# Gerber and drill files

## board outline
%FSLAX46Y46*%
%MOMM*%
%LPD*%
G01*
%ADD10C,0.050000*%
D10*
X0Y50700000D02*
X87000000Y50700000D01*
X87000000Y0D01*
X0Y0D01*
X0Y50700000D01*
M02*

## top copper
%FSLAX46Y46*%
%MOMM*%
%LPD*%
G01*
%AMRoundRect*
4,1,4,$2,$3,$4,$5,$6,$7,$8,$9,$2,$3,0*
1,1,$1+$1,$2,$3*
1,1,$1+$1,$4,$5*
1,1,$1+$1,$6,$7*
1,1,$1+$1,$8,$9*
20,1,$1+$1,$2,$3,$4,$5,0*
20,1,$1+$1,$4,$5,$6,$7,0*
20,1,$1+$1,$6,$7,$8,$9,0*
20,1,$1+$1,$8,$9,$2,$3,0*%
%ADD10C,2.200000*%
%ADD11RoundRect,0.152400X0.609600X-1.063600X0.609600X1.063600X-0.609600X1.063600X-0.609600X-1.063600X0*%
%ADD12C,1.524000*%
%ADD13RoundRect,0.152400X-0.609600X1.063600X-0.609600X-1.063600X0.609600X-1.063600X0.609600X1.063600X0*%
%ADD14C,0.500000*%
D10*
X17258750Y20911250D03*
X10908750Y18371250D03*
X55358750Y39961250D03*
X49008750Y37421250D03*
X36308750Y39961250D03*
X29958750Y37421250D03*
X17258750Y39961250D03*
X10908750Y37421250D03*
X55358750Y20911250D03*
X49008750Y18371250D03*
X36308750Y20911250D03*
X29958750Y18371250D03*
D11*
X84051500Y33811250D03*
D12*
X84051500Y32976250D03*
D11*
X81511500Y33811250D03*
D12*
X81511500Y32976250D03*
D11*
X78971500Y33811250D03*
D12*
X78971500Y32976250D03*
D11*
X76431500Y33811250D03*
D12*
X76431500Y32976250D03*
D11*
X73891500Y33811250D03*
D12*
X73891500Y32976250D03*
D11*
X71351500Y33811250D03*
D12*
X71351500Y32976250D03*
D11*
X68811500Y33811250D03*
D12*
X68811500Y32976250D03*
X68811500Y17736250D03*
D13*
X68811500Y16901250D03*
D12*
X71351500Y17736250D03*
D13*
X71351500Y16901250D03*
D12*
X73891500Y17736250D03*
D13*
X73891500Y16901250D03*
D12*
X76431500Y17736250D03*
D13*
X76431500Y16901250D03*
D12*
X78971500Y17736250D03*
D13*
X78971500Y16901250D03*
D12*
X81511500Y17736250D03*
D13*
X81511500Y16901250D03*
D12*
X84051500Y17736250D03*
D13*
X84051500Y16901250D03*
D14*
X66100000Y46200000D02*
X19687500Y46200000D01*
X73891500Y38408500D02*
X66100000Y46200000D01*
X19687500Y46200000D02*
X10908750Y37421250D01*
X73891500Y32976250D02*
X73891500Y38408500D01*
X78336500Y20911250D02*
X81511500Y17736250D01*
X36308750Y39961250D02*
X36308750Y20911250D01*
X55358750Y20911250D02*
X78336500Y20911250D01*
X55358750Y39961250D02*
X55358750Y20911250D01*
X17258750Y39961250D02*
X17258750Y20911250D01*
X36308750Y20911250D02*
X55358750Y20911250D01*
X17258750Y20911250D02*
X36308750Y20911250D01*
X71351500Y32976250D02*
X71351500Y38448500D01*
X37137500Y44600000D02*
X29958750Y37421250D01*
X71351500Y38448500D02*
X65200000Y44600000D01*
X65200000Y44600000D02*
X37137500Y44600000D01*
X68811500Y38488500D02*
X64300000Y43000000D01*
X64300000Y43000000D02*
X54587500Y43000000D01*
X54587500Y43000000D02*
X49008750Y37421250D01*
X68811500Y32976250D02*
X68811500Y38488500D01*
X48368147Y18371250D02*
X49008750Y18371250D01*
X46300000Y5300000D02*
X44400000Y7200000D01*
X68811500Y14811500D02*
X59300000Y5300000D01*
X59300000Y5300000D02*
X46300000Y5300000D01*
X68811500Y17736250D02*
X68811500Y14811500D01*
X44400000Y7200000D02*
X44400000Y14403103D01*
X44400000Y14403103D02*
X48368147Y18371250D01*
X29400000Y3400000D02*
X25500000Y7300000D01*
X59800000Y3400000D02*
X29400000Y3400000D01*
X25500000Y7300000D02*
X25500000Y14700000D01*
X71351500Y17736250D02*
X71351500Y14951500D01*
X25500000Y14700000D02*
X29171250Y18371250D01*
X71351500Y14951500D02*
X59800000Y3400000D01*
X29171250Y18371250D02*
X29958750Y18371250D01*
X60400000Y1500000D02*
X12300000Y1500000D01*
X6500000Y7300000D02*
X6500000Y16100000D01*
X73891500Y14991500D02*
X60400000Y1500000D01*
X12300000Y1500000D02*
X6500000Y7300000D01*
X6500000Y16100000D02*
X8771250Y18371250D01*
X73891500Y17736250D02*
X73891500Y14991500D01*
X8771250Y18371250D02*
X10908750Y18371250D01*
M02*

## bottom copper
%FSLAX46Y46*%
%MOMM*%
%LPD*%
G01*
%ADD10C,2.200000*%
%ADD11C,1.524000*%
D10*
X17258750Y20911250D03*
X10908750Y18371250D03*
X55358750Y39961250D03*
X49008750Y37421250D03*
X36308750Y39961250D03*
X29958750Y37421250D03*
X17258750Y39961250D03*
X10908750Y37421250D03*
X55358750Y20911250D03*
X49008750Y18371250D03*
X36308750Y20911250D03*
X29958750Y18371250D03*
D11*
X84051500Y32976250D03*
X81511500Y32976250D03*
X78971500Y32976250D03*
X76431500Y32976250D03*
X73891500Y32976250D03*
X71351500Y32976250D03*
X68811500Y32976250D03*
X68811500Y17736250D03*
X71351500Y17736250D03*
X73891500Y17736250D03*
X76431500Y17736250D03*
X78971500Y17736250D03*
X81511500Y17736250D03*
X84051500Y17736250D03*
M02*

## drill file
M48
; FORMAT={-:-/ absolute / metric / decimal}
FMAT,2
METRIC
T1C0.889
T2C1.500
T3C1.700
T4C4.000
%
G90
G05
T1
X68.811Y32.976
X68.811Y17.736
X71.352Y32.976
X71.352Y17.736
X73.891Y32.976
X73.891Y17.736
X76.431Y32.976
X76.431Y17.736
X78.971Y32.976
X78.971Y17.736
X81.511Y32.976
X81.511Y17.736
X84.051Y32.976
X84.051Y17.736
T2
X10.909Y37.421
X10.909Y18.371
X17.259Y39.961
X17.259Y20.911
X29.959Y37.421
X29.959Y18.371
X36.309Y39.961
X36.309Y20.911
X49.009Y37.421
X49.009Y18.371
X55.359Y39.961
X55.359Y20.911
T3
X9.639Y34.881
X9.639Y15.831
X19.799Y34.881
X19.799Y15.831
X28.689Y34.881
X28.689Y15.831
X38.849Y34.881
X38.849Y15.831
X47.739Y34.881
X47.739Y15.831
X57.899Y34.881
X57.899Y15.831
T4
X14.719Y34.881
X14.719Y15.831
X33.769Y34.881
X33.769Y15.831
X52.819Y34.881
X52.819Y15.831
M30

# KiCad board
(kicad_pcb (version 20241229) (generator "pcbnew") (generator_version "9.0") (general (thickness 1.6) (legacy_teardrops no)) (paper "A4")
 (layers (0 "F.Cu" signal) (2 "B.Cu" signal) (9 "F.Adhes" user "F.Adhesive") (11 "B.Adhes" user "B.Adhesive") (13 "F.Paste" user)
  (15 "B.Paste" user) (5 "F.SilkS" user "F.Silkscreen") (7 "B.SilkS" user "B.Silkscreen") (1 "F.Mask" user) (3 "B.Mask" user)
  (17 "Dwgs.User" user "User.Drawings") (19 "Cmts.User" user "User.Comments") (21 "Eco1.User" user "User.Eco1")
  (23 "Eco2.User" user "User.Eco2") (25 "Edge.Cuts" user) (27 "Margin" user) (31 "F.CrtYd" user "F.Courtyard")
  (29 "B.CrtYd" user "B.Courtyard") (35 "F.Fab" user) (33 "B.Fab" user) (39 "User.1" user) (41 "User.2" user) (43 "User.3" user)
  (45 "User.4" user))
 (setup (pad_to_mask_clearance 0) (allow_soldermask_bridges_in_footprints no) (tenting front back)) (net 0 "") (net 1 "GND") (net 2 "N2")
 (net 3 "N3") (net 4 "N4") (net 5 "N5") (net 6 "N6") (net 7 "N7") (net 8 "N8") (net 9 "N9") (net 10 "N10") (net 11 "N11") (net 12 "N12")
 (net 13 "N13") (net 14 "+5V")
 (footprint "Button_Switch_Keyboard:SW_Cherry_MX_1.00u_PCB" (layer "F.Cu") (at 17.25875 -20.91125)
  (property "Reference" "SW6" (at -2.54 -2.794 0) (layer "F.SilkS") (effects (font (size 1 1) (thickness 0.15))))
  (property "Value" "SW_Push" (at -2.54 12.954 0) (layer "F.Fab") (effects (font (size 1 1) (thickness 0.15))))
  (pad "" np_thru_hole circle (at -7.62 5.08) (size 1.7 1.7) (drill 1.7) (layers "*.Cu" "*.Mask"))
  (pad "" np_thru_hole circle (at -2.54 5.08) (size 4 4) (drill 4) (layers "*.Cu" "*.Mask"))
  (pad "" np_thru_hole circle (at 2.54 5.08) (size 1.7 1.7) (drill 1.7) (layers "*.Cu" "*.Mask"))
  (pad "1" thru_hole circle (at 0 0) (size 2.2 2.2) (drill 1.5) (layers "*.Cu" "*.Mask") (remove_unused_layers no) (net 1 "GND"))
  (pad "2" thru_hole circle (at -6.35 2.54) (size 2.2 2.2) (drill 1.5) (layers "*.Cu" "*.Mask") (remove_unused_layers no) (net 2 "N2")))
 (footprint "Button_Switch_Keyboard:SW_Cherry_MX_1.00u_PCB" (layer "F.Cu") (at 55.35875 -39.96125)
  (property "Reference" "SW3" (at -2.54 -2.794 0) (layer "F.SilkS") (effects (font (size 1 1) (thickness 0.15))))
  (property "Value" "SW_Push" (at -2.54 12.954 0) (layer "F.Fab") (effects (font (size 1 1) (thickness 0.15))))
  (pad "" np_thru_hole circle (at -7.62 5.08) (size 1.7 1.7) (drill 1.7) (layers "*.Cu" "*.Mask"))
  (pad "" np_thru_hole circle (at -2.54 5.08) (size 4 4) (drill 4) (layers "*.Cu" "*.Mask"))
  (pad "" np_thru_hole circle (at 2.54 5.08) (size 1.7 1.7) (drill 1.7) (layers "*.Cu" "*.Mask"))
  (pad "1" thru_hole circle (at 0 0) (size 2.2 2.2) (drill 1.5) (layers "*.Cu" "*.Mask") (remove_unused_layers no) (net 1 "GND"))
  (pad "2" thru_hole circle (at -6.35 2.54) (size 2.2 2.2) (drill 1.5) (layers "*.Cu" "*.Mask") (remove_unused_layers no) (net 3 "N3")))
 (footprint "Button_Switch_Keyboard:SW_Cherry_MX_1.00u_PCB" (layer "F.Cu") (at 36.30875 -39.96125)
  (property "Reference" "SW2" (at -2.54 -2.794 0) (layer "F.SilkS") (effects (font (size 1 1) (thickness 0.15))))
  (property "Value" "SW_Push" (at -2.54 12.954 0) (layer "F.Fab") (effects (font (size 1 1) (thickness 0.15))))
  (pad "" np_thru_hole circle (at -7.62 5.08) (size 1.7 1.7) (drill 1.7) (layers "*.Cu" "*.Mask"))
  (pad "" np_thru_hole circle (at -2.54 5.08) (size 4 4) (drill 4) (layers "*.Cu" "*.Mask"))
  (pad "" np_thru_hole circle (at 2.54 5.08) (size 1.7 1.7) (drill 1.7) (layers "*.Cu" "*.Mask"))
  (pad "1" thru_hole circle (at 0 0) (size 2.2 2.2) (drill 1.5) (layers "*.Cu" "*.Mask") (remove_unused_layers no) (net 1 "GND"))
  (pad "2" thru_hole circle (at -6.35 2.54) (size 2.2 2.2) (drill 1.5) (layers "*.Cu" "*.Mask") (remove_unused_layers no) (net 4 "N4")))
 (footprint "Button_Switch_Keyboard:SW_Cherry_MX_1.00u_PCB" (layer "F.Cu") (at 17.25875 -39.96125)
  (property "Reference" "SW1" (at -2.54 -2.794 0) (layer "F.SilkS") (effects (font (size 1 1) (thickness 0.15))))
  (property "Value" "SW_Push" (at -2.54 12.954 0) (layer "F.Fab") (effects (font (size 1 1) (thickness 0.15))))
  (pad "" np_thru_hole circle (at -7.62 5.08) (size 1.7 1.7) (drill 1.7) (layers "*.Cu" "*.Mask"))
  (pad "" np_thru_hole circle (at -2.54 5.08) (size 4 4) (drill 4) (layers "*.Cu" "*.Mask"))
  (pad "" np_thru_hole circle (at 2.54 5.08) (size 1.7 1.7) (drill 1.7) (layers "*.Cu" "*.Mask"))
  (pad "1" thru_hole circle (at 0 0) (size 2.2 2.2) (drill 1.5) (layers "*.Cu" "*.Mask") (remove_unused_layers no) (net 1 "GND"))
  (pad "2" thru_hole circle (at -6.35 2.54) (size 2.2 2.2) (drill 1.5) (layers "*.Cu" "*.Mask") (remove_unused_layers no) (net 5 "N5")))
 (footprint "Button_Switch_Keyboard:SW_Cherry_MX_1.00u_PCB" (layer "F.Cu") (at 55.35875 -20.91125)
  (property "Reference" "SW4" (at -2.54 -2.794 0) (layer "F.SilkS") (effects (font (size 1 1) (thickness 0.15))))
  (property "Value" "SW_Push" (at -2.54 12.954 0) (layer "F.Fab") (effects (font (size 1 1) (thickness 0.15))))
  (pad "" np_thru_hole circle (at -7.62 5.08) (size 1.7 1.7) (drill 1.7) (layers "*.Cu" "*.Mask"))
  (pad "" np_thru_hole circle (at -2.54 5.08) (size 4 4) (drill 4) (layers "*.Cu" "*.Mask"))
  (pad "" np_thru_hole circle (at 2.54 5.08) (size 1.7 1.7) (drill 1.7) (layers "*.Cu" "*.Mask"))
  (pad "1" thru_hole circle (at 0 0) (size 2.2 2.2) (drill 1.5) (layers "*.Cu" "*.Mask") (remove_unused_layers no) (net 1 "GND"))
  (pad "2" thru_hole circle (at -6.35 2.54) (size 2.2 2.2) (drill 1.5) (layers "*.Cu" "*.Mask") (remove_unused_layers no) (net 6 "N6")))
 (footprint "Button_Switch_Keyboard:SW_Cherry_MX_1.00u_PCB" (layer "F.Cu") (at 36.30875 -20.91125)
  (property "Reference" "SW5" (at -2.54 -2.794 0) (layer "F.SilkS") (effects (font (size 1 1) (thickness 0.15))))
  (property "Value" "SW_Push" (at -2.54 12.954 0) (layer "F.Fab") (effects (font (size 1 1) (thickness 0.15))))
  (pad "" np_thru_hole circle (at -7.62 5.08) (size 1.7 1.7) (drill 1.7) (layers "*.Cu" "*.Mask"))
  (pad "" np_thru_hole circle (at -2.54 5.08) (size 4 4) (drill 4) (layers "*.Cu" "*.Mask"))
  (pad "" np_thru_hole circle (at 2.54 5.08) (size 1.7 1.7) (drill 1.7) (layers "*.Cu" "*.Mask"))
  (pad "1" thru_hole circle (at 0 0) (size 2.2 2.2) (drill 1.5) (layers "*.Cu" "*.Mask") (remove_unused_layers no) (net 1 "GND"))
  (pad "2" thru_hole circle (at -6.35 2.54) (size 2.2 2.2) (drill 1.5) (layers "*.Cu" "*.Mask") (remove_unused_layers no) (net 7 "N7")))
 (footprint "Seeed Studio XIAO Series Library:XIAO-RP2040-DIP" (layer "F.Cu") (at 76.4315 -25.35625 -90)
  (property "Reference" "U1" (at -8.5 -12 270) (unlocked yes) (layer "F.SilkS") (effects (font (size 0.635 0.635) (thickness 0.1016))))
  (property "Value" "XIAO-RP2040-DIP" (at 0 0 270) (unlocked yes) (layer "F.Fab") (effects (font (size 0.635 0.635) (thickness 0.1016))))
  (pad "1" smd roundrect (at -8.455 -7.62 90) (size 2.432 1.524) (layers "F.Cu" "F.Mask") (roundrect_rratio 0.1) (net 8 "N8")
   (thermal_bridge_angle 45))
  (pad "1" thru_hole circle (at -7.62 -7.62 90) (size 1.524 1.524) (drill 0.889) (layers "*.Cu" "*.Mask") (remove_unused_layers no)
   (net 8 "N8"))
  (pad "2" smd roundrect (at -8.455 -5.08 90) (size 2.432 1.524) (layers "F.Cu" "F.Mask") (roundrect_rratio 0.1) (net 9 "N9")
   (thermal_bridge_angle 45))
  (pad "2" thru_hole circle (at -7.62 -5.08 90) (size 1.524 1.524) (drill 0.889) (layers "*.Cu" "*.Mask") (remove_unused_layers no)
   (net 9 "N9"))
  (pad "3" smd roundrect (at -8.455 -2.54 90) (size 2.432 1.524) (layers "F.Cu" "F.Mask") (roundrect_rratio 0.1) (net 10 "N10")
   (thermal_bridge_angle 45))
  (pad "3" thru_hole circle (at -7.62 -2.54 90) (size 1.524 1.524) (drill 0.889) (layers "*.Cu" "*.Mask") (remove_unused_layers no)
   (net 10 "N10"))
  (pad "4" smd roundrect (at -8.455 0 90) (size 2.432 1.524) (layers "F.Cu" "F.Mask") (roundrect_rratio 0.1) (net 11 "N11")
   (thermal_bridge_angle 45))
  (pad "4" thru_hole circle (at -7.62 0 90) (size 1.524 1.524) (drill 0.889) (layers "*.Cu" "*.Mask") (remove_unused_layers no)
   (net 11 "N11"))
  (pad "5" smd roundrect (at -8.455 2.54 90) (size 2.432 1.524) (layers "F.Cu" "F.Mask") (roundrect_rratio 0.1) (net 5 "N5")
   (thermal_bridge_angle 45))
  (pad "5" thru_hole circle (at -7.62 2.54 90) (size 1.524 1.524) (drill 0.889) (layers "*.Cu" "*.Mask") (remove_unused_layers no)
   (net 5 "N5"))
  (pad "6" smd roundrect (at -8.455 5.08 90) (size 2.432 1.524) (layers "F.Cu" "F.Mask") (roundrect_rratio 0.1) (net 4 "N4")
   (thermal_bridge_angle 45))
  (pad "6" thru_hole circle (at -7.62 5.08 90) (size 1.524 1.524) (drill 0.889) (layers "*.Cu" "*.Mask") (remove_unused_layers no)
   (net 4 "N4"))
  (pad "7" smd roundrect (at -8.455 7.62 90) (size 2.432 1.524) (layers "F.Cu" "F.Mask") (roundrect_rratio 0.1) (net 3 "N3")
   (thermal_bridge_angle 45))
  (pad "7" thru_hole circle (at -7.62 7.62 90) (size 1.524 1.524) (drill 0.889) (layers "*.Cu" "*.Mask") (remove_unused_layers no)
   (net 3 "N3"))
  (pad "8" thru_hole circle (at 7.62 7.62 270) (size 1.524 1.524) (drill 0.889) (layers "*.Cu" "*.Mask") (remove_unused_layers no)
   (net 6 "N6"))
  (pad "8" smd roundrect (at 8.455 7.62 270) (size 2.432 1.524) (layers "F.Cu" "F.Mask") (roundrect_rratio 0.1) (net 6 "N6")
   (thermal_bridge_angle 45))
  (pad "9" thru_hole circle (at 7.62 5.08 270) (size 1.524 1.524) (drill 0.889) (layers "*.Cu" "*.Mask") (remove_unused_layers no)
   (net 7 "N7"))
  (pad "9" smd roundrect (at 8.455 5.08 270) (size 2.432 1.524) (layers "F.Cu" "F.Mask") (roundrect_rratio 0.1) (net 7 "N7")
   (thermal_bridge_angle 45))
  (pad "10" thru_hole circle (at 7.62 2.54 270) (size 1.524 1.524) (drill 0.889) (layers "*.Cu" "*.Mask") (remove_unused_layers no)
   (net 2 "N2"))
  (pad "10" smd roundrect (at 8.455 2.54 270) (size 2.432 1.524) (layers "F.Cu" "F.Mask") (roundrect_rratio 0.1) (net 2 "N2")
   (thermal_bridge_angle 45))
  (pad "11" thru_hole circle (at 7.62 0 270) (size 1.524 1.524) (drill 0.889) (layers "*.Cu" "*.Mask") (remove_unused_layers no)
   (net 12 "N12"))
  (pad "11" smd roundrect (at 8.455 0 270) (size 2.432 1.524) (layers "F.Cu" "F.Mask") (roundrect_rratio 0.1) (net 12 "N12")
   (thermal_bridge_angle 45))
  (pad "12" thru_hole circle (at 7.62 -2.54 270) (size 1.524 1.524) (drill 0.889) (layers "*.Cu" "*.Mask") (remove_unused_layers no)
   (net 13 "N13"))
  (pad "12" smd roundrect (at 8.455 -2.54 270) (size 2.432 1.524) (layers "F.Cu" "F.Mask") (roundrect_rratio 0.1) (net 13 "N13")
   (thermal_bridge_angle 45))
  (pad "13" thru_hole circle (at 7.62 -5.08 270) (size 1.524 1.524) (drill 0.889) (layers "*.Cu" "*.Mask") (remove_unused_layers no)
   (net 1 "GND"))
  (pad "13" smd roundrect (at 8.455 -5.08 270) (size 2.432 1.524) (layers "F.Cu" "F.Mask") (roundrect_rratio 0.1) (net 1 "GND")
   (thermal_bridge_angle 45))
  (pad "14" thru_hole circle (at 7.62 -7.62 270) (size 1.524 1.524) (drill 0.889) (layers "*.Cu" "*.Mask") (remove_unused_layers no)
   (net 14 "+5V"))
  (pad "14" smd roundrect (at 8.455 -7.62 270) (size 2.432 1.524) (layers "F.Cu" "F.Mask") (roundrect_rratio 0.1) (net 14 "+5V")
   (thermal_bridge_angle 45)))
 (gr_rect (start 0 -50.7) (end 87 0) (stroke (width 0.05) (type default)) (fill no) (layer "Edge.Cuts"))
 (segment (start 66.1 -46.2) (end 19.6875 -46.2) (width 0.5) (layer "F.Cu") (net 5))
 (segment (start 73.8915 -38.4085) (end 66.1 -46.2) (width 0.5) (layer "F.Cu") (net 5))
 (segment (start 19.6875 -46.2) (end 10.90875 -37.42125) (width 0.5) (layer "F.Cu") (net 5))
 (segment (start 73.8915 -32.97625) (end 73.8915 -38.4085) (width 0.5) (layer "F.Cu") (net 5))
 (segment (start 78.3365 -20.91125) (end 81.5115 -17.73625) (width 0.5) (layer "F.Cu") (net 1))
 (segment (start 36.30875 -39.96125) (end 36.30875 -20.91125) (width 0.5) (layer "F.Cu") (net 1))
 (segment (start 55.35875 -20.91125) (end 78.3365 -20.91125) (width 0.5) (layer "F.Cu") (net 1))
 (segment (start 55.35875 -39.96125) (end 55.35875 -20.91125) (width 0.5) (layer "F.Cu") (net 1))
 (segment (start 17.25875 -39.96125) (end 17.25875 -20.91125) (width 0.5) (layer "F.Cu") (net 1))
 (segment (start 36.30875 -20.91125) (end 55.35875 -20.91125) (width 0.5) (layer "F.Cu") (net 1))
 (segment (start 17.25875 -20.91125) (end 36.30875 -20.91125) (width 0.5) (layer "F.Cu") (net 1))
 (segment (start 71.3515 -32.97625) (end 71.3515 -38.4485) (width 0.5) (layer "F.Cu") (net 4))
 (segment (start 37.1375 -44.6) (end 29.95875 -37.42125) (width 0.5) (layer "F.Cu") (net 4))
 (segment (start 71.3515 -38.4485) (end 65.2 -44.6) (width 0.5) (layer "F.Cu") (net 4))
 (segment (start 65.2 -44.6) (end 37.1375 -44.6) (width 0.5) (layer "F.Cu") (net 4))
 (segment (start 68.8115 -38.4885) (end 64.3 -43) (width 0.5) (layer "F.Cu") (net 3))
 (segment (start 64.3 -43) (end 54.5875 -43) (width 0.5) (layer "F.Cu") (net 3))
 (segment (start 54.5875 -43) (end 49.00875 -37.42125) (width 0.5) (layer "F.Cu") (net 3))
 (segment (start 68.8115 -32.97625) (end 68.8115 -38.4885) (width 0.5) (layer "F.Cu") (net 3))
 (segment (start 48.368147 -18.37125) (end 49.00875 -18.37125) (width 0.5) (layer "F.Cu") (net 6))
 (segment (start 46.3 -5.3) (end 44.4 -7.2) (width 0.5) (layer "F.Cu") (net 6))
 (segment (start 68.8115 -14.8115) (end 59.3 -5.3) (width 0.5) (layer "F.Cu") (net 6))
 (segment (start 59.3 -5.3) (end 46.3 -5.3) (width 0.5) (layer "F.Cu") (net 6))
 (segment (start 68.8115 -17.73625) (end 68.8115 -14.8115) (width 0.5) (layer "F.Cu") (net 6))
 (segment (start 44.4 -7.2) (end 44.4 -14.403103) (width 0.5) (layer "F.Cu") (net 6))
 (segment (start 44.4 -14.403103) (end 48.368147 -18.37125) (width 0.5) (layer "F.Cu") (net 6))
 (segment (start 29.4 -3.4) (end 25.5 -7.3) (width 0.5) (layer "F.Cu") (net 7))
 (segment (start 59.8 -3.4) (end 29.4 -3.4) (width 0.5) (layer "F.Cu") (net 7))
 (segment (start 25.5 -7.3) (end 25.5 -14.7) (width 0.5) (layer "F.Cu") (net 7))
 (segment (start 71.3515 -17.73625) (end 71.3515 -14.9515) (width 0.5) (layer "F.Cu") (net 7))
 (segment (start 25.5 -14.7) (end 29.17125 -18.37125) (width 0.5) (layer "F.Cu") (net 7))
 (segment (start 71.3515 -14.9515) (end 59.8 -3.4) (width 0.5) (layer "F.Cu") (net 7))
 (segment (start 29.17125 -18.37125) (end 29.95875 -18.37125) (width 0.5) (layer "F.Cu") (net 7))
 (segment (start 60.4 -1.5) (end 12.3 -1.5) (width 0.5) (layer "F.Cu") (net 2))
 (segment (start 6.5 -7.3) (end 6.5 -16.1) (width 0.5) (layer "F.Cu") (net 2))
 (segment (start 73.8915 -14.9915) (end 60.4 -1.5) (width 0.5) (layer "F.Cu") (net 2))
 (segment (start 12.3 -1.5) (end 6.5 -7.3) (width 0.5) (layer "F.Cu") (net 2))
 (segment (start 6.5 -16.1) (end 8.77125 -18.37125) (width 0.5) (layer "F.Cu") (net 2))
 (segment (start 73.8915 -17.73625) (end 73.8915 -14.9915) (width 0.5) (layer "F.Cu") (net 2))
 (segment (start 8.77125 -18.37125) (end 10.90875 -18.37125) (width 0.5) (layer "F.Cu") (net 2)))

